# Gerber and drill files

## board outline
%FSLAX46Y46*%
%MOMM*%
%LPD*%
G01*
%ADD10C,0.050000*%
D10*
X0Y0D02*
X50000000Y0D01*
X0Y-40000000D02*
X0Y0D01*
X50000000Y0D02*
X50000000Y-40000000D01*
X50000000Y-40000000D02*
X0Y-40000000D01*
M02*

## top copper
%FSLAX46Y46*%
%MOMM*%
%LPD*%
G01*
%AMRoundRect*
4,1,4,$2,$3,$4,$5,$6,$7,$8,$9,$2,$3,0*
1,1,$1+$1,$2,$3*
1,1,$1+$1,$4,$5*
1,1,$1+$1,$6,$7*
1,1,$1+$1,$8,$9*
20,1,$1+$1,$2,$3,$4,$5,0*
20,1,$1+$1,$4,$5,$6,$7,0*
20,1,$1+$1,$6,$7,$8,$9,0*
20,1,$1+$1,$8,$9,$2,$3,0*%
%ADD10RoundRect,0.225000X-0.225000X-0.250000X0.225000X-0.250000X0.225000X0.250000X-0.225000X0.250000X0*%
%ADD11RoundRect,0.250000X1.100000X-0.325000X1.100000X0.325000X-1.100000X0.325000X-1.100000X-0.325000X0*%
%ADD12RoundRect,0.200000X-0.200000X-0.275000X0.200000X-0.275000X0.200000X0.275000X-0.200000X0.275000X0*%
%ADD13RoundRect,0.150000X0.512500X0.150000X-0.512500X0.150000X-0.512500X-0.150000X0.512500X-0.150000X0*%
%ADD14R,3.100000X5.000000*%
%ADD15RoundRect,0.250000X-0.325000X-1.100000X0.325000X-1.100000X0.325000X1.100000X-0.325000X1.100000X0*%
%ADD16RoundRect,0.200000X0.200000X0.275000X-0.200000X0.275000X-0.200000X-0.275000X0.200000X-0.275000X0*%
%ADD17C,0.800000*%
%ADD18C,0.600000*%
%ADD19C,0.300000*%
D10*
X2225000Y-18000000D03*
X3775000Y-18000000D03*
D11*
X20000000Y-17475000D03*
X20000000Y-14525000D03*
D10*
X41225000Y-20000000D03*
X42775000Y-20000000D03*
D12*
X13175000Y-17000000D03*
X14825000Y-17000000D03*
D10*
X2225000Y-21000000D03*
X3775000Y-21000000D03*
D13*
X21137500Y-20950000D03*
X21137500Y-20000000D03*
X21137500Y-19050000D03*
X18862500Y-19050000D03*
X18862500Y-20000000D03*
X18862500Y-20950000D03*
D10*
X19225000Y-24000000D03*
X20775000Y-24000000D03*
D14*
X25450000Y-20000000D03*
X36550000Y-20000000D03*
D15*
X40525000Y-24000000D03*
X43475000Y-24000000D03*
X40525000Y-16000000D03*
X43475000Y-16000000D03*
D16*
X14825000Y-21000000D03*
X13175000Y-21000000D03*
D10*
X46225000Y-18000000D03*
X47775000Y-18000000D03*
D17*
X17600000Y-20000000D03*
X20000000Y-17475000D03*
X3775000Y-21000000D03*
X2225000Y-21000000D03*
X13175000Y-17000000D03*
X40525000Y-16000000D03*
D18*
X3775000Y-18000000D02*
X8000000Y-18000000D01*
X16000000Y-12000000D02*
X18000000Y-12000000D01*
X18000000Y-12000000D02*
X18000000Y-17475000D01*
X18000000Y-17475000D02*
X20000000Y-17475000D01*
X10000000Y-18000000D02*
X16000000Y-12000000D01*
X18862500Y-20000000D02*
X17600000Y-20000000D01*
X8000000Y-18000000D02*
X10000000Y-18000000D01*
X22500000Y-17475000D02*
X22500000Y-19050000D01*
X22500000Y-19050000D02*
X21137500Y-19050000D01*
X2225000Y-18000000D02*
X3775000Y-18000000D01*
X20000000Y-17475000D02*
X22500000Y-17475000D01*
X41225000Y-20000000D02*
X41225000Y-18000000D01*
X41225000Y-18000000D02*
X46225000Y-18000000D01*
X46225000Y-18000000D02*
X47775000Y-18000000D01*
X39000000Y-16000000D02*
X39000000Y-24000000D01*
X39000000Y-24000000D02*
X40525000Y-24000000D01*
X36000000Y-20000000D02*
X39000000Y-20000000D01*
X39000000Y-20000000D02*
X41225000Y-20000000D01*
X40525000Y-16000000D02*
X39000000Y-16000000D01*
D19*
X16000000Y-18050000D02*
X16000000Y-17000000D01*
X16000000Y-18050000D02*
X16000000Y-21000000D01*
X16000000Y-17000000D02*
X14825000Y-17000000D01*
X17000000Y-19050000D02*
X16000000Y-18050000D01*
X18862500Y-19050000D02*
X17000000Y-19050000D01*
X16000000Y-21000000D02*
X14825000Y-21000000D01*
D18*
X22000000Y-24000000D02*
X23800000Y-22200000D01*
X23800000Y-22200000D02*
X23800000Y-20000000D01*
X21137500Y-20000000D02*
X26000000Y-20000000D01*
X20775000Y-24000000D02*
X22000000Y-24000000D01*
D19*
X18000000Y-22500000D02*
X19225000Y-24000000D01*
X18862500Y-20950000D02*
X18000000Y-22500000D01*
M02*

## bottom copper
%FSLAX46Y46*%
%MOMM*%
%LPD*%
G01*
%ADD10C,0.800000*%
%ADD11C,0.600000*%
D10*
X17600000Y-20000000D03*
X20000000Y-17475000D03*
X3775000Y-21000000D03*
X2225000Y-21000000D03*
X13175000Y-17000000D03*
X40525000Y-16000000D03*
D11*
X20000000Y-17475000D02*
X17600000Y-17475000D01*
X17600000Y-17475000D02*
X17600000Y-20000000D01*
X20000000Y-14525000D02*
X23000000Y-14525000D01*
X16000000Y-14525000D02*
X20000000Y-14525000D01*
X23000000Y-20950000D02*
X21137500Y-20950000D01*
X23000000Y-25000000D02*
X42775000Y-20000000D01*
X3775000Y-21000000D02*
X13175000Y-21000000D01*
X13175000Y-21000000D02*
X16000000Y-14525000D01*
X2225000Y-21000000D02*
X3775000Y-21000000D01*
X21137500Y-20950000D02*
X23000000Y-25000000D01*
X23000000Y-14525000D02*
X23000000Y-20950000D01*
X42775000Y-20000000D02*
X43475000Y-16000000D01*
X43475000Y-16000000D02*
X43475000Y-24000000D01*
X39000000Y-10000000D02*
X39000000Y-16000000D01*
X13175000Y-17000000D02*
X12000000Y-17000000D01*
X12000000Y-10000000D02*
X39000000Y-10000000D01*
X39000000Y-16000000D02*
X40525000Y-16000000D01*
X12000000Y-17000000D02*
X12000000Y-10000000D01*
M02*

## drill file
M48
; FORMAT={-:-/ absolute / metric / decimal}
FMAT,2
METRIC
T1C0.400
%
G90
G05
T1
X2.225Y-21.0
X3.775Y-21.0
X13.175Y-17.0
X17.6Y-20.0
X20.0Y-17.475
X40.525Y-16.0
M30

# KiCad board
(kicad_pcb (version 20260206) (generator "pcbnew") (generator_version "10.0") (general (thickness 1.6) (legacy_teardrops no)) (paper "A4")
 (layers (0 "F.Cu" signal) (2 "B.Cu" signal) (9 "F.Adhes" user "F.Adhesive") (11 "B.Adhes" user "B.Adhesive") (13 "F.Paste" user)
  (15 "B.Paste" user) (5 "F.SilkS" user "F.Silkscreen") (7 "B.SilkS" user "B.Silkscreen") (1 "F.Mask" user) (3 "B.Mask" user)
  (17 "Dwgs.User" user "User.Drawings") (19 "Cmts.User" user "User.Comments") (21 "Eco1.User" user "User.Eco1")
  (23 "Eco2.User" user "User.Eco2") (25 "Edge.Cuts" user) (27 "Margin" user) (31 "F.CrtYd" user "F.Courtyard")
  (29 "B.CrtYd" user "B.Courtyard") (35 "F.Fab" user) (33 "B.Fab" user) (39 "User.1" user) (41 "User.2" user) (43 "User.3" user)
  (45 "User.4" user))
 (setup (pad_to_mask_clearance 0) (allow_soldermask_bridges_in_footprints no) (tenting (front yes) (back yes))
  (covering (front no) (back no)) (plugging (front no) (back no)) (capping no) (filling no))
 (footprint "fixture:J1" (layer "F.Cu") (at 3 18)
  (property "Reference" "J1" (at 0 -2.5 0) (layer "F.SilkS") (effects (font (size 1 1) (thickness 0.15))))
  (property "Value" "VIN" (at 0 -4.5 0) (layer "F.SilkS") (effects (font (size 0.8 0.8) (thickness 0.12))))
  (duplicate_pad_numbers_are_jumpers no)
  (pad "1" smd roundrect (at -0.775 0) (size 0.9 0.95) (layers "F.Cu" "F.Mask" "F.Paste") (roundrect_rratio 0.25) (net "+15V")
   (thermal_bridge_angle 45))
  (pad "2" smd roundrect (at 0.775 0) (size 0.9 0.95) (layers "F.Cu" "F.Mask" "F.Paste") (roundrect_rratio 0.25) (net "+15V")
   (thermal_bridge_angle 45)))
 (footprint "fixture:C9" (layer "F.Cu") (at 20 16 90)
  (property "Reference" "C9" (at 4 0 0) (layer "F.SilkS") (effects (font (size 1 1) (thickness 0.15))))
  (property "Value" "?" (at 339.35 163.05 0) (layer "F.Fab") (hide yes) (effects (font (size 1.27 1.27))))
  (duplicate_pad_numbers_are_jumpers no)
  (pad "1" smd roundrect (at -1.475 0 90) (size 1.15 2.7) (layers "F.Cu" "F.Mask" "F.Paste") (roundrect_rratio 0.217391) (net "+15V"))
  (pad "2" smd roundrect (at 1.475 0 90) (size 1.15 2.7) (layers "F.Cu" "F.Mask" "F.Paste") (roundrect_rratio 0.217391) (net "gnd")))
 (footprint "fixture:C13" (layer "F.Cu") (at 42 20)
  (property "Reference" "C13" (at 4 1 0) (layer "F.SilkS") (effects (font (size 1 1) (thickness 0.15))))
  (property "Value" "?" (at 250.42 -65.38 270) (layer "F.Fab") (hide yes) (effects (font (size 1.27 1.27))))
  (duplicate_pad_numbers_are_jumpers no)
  (pad "1" smd roundrect (at -0.775 0) (size 0.9 0.95) (layers "F.Cu" "F.Mask" "F.Paste") (roundrect_rratio 0.25) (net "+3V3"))
  (pad "2" smd roundrect (at 0.775 0) (size 0.9 0.95) (layers "F.Cu" "F.Mask" "F.Paste") (roundrect_rratio 0.25) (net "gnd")))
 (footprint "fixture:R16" (layer "F.Cu") (at 14 17)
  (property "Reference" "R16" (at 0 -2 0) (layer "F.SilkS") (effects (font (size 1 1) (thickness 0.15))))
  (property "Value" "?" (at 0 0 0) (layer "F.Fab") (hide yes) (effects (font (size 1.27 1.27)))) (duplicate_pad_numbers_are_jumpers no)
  (pad "1" smd roundrect (at -0.825 0) (size 0.8 0.95) (layers "F.Cu" "F.Mask" "F.Paste") (roundrect_rratio 0.25) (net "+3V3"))
  (pad "2" smd roundrect (at 0.825 0) (size 0.8 0.95) (layers "F.Cu" "F.Mask" "F.Paste") (roundrect_rratio 0.25) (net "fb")))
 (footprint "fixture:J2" (layer "F.Cu") (at 3 21)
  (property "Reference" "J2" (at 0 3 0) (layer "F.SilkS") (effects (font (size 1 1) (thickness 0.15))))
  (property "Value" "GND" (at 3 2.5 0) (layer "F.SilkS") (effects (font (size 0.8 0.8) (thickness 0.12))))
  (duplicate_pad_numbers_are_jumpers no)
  (pad "1" smd roundrect (at -0.775 0) (size 0.9 0.95) (layers "F.Cu" "F.Mask" "F.Paste") (roundrect_rratio 0.25) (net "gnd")
   (thermal_bridge_angle 45))
  (pad "2" smd roundrect (at 0.775 0) (size 0.9 0.95) (layers "F.Cu" "F.Mask" "F.Paste") (roundrect_rratio 0.25) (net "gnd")
   (thermal_bridge_angle 45)))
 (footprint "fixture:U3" (layer "F.Cu") (at 20 20 180)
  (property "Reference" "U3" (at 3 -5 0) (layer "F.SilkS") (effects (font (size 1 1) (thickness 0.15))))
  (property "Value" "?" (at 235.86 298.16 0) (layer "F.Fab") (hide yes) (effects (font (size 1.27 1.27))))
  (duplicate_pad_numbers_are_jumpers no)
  (pad "1" smd roundrect (at -1.1375 -0.95 180) (size 1.325 0.6) (layers "F.Cu" "F.Mask" "F.Paste") (roundrect_rratio 0.25) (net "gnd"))
  (pad "2" smd roundrect (at -1.1375 0 180) (size 1.325 0.6) (layers "F.Cu" "F.Mask" "F.Paste") (roundrect_rratio 0.25) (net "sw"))
  (pad "3" smd roundrect (at -1.1375 0.95 180) (size 1.325 0.6) (layers "F.Cu" "F.Mask" "F.Paste") (roundrect_rratio 0.25) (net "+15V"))
  (pad "4" smd roundrect (at 1.1375 0.95 180) (size 1.325 0.6) (layers "F.Cu" "F.Mask" "F.Paste") (roundrect_rratio 0.25) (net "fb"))
  (pad "5" smd roundrect (at 1.1375 0 180) (size 1.325 0.6) (layers "F.Cu" "F.Mask" "F.Paste") (roundrect_rratio 0.25) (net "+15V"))
  (pad "6" smd roundrect (at 1.1375 -0.95 180) (size 1.325 0.6) (layers "F.Cu" "F.Mask" "F.Paste") (roundrect_rratio 0.25) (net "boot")))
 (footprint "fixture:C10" (layer "F.Cu") (at 20 24)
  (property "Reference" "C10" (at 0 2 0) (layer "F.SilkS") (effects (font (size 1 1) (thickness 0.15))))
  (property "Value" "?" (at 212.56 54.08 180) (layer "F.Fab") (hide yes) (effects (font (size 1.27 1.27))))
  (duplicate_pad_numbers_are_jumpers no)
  (pad "1" smd roundrect (at -0.775 0) (size 0.9 0.95) (layers "F.Cu" "F.Mask" "F.Paste") (roundrect_rratio 0.25) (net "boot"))
  (pad "2" smd roundrect (at 0.775 0) (size 0.9 0.95) (layers "F.Cu" "F.Mask" "F.Paste") (roundrect_rratio 0.25) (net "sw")))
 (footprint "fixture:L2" (layer "F.Cu") (at 31 20)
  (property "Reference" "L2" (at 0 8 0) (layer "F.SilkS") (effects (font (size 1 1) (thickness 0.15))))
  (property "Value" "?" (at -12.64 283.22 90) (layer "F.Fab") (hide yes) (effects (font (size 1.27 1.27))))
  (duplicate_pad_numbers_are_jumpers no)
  (pad "1" smd rect (at -5.55 0) (size 3.1 5) (layers "F.Cu" "F.Mask" "F.Paste") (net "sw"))
  (pad "2" smd rect (at 5.55 0) (size 3.1 5) (layers "F.Cu" "F.Mask" "F.Paste") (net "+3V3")))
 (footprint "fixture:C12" (layer "F.Cu") (at 42 24)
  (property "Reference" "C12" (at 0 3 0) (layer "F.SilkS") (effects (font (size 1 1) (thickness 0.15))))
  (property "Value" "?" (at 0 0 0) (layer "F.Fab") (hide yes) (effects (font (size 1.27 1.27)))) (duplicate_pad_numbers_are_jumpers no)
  (pad "1" smd roundrect (at -1.475 0) (size 1.15 2.7) (layers "F.Cu" "F.Mask" "F.Paste") (roundrect_rratio 0.217391) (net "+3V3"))
  (pad "2" smd roundrect (at 1.475 0) (size 1.15 2.7) (layers "F.Cu" "F.Mask" "F.Paste") (roundrect_rratio 0.217391) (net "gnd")))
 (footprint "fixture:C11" (layer "F.Cu") (at 42 16)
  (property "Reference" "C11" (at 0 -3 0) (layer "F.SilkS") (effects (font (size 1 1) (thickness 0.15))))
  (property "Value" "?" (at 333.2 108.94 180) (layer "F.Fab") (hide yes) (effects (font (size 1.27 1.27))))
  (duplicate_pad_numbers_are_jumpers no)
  (pad "1" smd roundrect (at -1.475 0) (size 1.15 2.7) (layers "F.Cu" "F.Mask" "F.Paste") (roundrect_rratio 0.217391) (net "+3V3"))
  (pad "2" smd roundrect (at 1.475 0) (size 1.15 2.7) (layers "F.Cu" "F.Mask" "F.Paste") (roundrect_rratio 0.217391) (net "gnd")))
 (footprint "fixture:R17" (layer "F.Cu") (at 14 21 180)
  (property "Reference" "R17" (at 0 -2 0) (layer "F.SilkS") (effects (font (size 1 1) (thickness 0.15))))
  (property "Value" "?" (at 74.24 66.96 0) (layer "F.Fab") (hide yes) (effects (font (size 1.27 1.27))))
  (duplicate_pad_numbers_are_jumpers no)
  (pad "1" smd roundrect (at -0.825 0 180) (size 0.8 0.95) (layers "F.Cu" "F.Mask" "F.Paste") (roundrect_rratio 0.25) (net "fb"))
  (pad "2" smd roundrect (at 0.825 0 180) (size 0.8 0.95) (layers "F.Cu" "F.Mask" "F.Paste") (roundrect_rratio 0.25) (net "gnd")))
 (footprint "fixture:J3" (layer "F.Cu") (at 47 18)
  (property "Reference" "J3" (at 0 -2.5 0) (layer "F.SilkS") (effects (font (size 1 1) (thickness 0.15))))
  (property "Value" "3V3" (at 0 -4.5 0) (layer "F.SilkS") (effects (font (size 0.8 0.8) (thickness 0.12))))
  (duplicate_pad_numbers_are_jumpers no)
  (pad "1" smd roundrect (at -0.775 0) (size 0.9 0.95) (layers "F.Cu" "F.Mask" "F.Paste") (roundrect_rratio 0.25) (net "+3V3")
   (thermal_bridge_angle 45))
  (pad "2" smd roundrect (at 0.775 0) (size 0.9 0.95) (layers "F.Cu" "F.Mask" "F.Paste") (roundrect_rratio 0.25) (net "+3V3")
   (thermal_bridge_angle 45)))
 (gr_line (start 0 0) (end 50 0) (stroke (width 0.05) (type default)) (layer "Edge.Cuts"))
 (gr_line (start 0 40) (end 0 0) (stroke (width 0.05) (type default)) (layer "Edge.Cuts"))
 (gr_line (start 50 0) (end 50 40) (stroke (width 0.05) (type default)) (layer "Edge.Cuts"))
 (gr_line (start 50 40) (end 0 40) (stroke (width 0.05) (type default)) (layer "Edge.Cuts"))
 (segment (start 3.775 18) (end 8 18) (width 0.6) (layer "F.Cu") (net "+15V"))
 (segment (start 16 12) (end 18 12) (width 0.6) (layer "F.Cu") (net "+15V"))
 (segment (start 18 12) (end 18 17.475) (width 0.6) (layer "F.Cu") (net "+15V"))
 (segment (start 18 17.475) (end 20 17.475) (width 0.6) (layer "F.Cu") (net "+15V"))
 (segment (start 10 18) (end 16 12) (width 0.6) (layer "F.Cu") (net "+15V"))
 (segment (start 18.8625 20) (end 17.6 20) (width 0.6) (layer "F.Cu") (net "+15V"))
 (segment (start 8 18) (end 10 18) (width 0.6) (layer "F.Cu") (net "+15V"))
 (segment (start 22.5 17.475) (end 22.5 19.05) (width 0.6) (layer "F.Cu") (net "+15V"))
 (segment (start 22.5 19.05) (end 21.1375 19.05) (width 0.6) (layer "F.Cu") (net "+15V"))
 (segment (start 2.225 18) (end 3.775 18) (width 0.6) (layer "F.Cu") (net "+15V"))
 (segment (start 20 17.475) (end 22.5 17.475) (width 0.6) (layer "F.Cu") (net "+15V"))
 (via (at 17.6 20) (size 0.8) (drill 0.4) (layers "F.Cu" "B.Cu") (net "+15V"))
 (via (at 20 17.475) (size 0.8) (drill 0.4) (layers "F.Cu" "B.Cu") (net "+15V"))
 (segment (start 20 17.475) (end 17.6 17.475) (width 0.6) (layer "B.Cu") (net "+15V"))
 (segment (start 17.6 17.475) (end 17.6 20) (width 0.6) (layer "B.Cu") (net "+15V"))
 (via (at 3.775 21) (size 0.8) (drill 0.4) (layers "F.Cu" "B.Cu") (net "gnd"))
 (via (at 2.225 21) (size 0.8) (drill 0.4) (layers "F.Cu" "B.Cu") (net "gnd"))
 (segment (start 20 14.525) (end 23 14.525) (width 0.6) (layer "B.Cu") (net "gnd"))
 (segment (start 16 14.525) (end 20 14.525) (width 0.6) (layer "B.Cu") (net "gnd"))
 (segment (start 23 20.95) (end 21.1375 20.95) (width 0.6) (layer "B.Cu") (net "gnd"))
 (segment (start 23 25) (end 42.775 20) (width 0.6) (layer "B.Cu") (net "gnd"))
 (segment (start 3.775 21) (end 13.175 21) (width 0.6) (layer "B.Cu") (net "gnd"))
 (segment (start 13.175 21) (end 16 14.525) (width 0.6) (layer "B.Cu") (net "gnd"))
 (segment (start 2.225 21) (end 3.775 21) (width 0.6) (layer "B.Cu") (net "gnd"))
 (segment (start 21.1375 20.95) (end 23 25) (width 0.6) (layer "B.Cu") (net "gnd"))
 (segment (start 23 14.525) (end 23 20.95) (width 0.6) (layer "B.Cu") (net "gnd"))
 (segment (start 42.775 20) (end 43.475 16) (width 0.6) (layer "B.Cu") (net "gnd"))
 (segment (start 43.475 16) (end 43.475 24) (width 0.6) (layer "B.Cu") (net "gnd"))
 (segment (start 41.225 20) (end 41.225 18) (width 0.6) (layer "F.Cu") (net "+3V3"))
 (segment (start 41.225 18) (end 46.225 18) (width 0.6) (layer "F.Cu") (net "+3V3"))
 (segment (start 46.225 18) (end 47.775 18) (width 0.6) (layer "F.Cu") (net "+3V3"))
 (segment (start 39 16) (end 39 24) (width 0.6) (layer "F.Cu") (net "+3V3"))
 (segment (start 39 24) (end 40.525 24) (width 0.6) (layer "F.Cu") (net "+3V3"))
 (segment (start 36 20) (end 39 20) (width 0.6) (layer "F.Cu") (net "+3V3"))
 (segment (start 39 20) (end 41.225 20) (width 0.6) (layer "F.Cu") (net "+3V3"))
 (segment (start 40.525 16) (end 39 16) (width 0.6) (layer "F.Cu") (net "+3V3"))
 (via (at 13.175 17) (size 0.8) (drill 0.4) (layers "F.Cu" "B.Cu") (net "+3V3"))
 (via (at 40.525 16) (size 0.8) (drill 0.4) (layers "F.Cu" "B.Cu") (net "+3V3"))
 (segment (start 39 10) (end 39 16) (width 0.6) (layer "B.Cu") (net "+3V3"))
 (segment (start 13.175 17) (end 12 17) (width 0.6) (layer "B.Cu") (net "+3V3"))
 (segment (start 12 10) (end 39 10) (width 0.6) (layer "B.Cu") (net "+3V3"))
 (segment (start 39 16) (end 40.525 16) (width 0.6) (layer "B.Cu") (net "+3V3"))
 (segment (start 12 17) (end 12 10) (width 0.6) (layer "B.Cu") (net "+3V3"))
 (segment (start 16 18.05) (end 16 17) (width 0.3) (layer "F.Cu") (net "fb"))
 (segment (start 16 18.05) (end 16 21) (width 0.3) (layer "F.Cu") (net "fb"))
 (segment (start 16 17) (end 14.825 17) (width 0.3) (layer "F.Cu") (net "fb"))
 (segment (start 17 19.05) (end 16 18.05) (width 0.3) (layer "F.Cu") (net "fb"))
 (segment (start 18.8625 19.05) (end 17 19.05) (width 0.3) (layer "F.Cu") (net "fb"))
 (segment (start 16 21) (end 14.825 21) (width 0.3) (layer "F.Cu") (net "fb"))
 (segment (start 22 24) (end 23.8 22.2) (width 0.6) (layer "F.Cu") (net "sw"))
 (segment (start 23.8 22.2) (end 23.8 20) (width 0.6) (layer "F.Cu") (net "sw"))
 (segment (start 21.1375 20) (end 26 20) (width 0.6) (layer "F.Cu") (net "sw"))
 (segment (start 20.775 24) (end 22 24) (width 0.6) (layer "F.Cu") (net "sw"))
 (segment (start 18 22.5) (end 19.225 24) (width 0.3) (layer "F.Cu") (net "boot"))
 (segment (start 18.8625 20.95) (end 18 22.5) (width 0.3) (layer "F.Cu") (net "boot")))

